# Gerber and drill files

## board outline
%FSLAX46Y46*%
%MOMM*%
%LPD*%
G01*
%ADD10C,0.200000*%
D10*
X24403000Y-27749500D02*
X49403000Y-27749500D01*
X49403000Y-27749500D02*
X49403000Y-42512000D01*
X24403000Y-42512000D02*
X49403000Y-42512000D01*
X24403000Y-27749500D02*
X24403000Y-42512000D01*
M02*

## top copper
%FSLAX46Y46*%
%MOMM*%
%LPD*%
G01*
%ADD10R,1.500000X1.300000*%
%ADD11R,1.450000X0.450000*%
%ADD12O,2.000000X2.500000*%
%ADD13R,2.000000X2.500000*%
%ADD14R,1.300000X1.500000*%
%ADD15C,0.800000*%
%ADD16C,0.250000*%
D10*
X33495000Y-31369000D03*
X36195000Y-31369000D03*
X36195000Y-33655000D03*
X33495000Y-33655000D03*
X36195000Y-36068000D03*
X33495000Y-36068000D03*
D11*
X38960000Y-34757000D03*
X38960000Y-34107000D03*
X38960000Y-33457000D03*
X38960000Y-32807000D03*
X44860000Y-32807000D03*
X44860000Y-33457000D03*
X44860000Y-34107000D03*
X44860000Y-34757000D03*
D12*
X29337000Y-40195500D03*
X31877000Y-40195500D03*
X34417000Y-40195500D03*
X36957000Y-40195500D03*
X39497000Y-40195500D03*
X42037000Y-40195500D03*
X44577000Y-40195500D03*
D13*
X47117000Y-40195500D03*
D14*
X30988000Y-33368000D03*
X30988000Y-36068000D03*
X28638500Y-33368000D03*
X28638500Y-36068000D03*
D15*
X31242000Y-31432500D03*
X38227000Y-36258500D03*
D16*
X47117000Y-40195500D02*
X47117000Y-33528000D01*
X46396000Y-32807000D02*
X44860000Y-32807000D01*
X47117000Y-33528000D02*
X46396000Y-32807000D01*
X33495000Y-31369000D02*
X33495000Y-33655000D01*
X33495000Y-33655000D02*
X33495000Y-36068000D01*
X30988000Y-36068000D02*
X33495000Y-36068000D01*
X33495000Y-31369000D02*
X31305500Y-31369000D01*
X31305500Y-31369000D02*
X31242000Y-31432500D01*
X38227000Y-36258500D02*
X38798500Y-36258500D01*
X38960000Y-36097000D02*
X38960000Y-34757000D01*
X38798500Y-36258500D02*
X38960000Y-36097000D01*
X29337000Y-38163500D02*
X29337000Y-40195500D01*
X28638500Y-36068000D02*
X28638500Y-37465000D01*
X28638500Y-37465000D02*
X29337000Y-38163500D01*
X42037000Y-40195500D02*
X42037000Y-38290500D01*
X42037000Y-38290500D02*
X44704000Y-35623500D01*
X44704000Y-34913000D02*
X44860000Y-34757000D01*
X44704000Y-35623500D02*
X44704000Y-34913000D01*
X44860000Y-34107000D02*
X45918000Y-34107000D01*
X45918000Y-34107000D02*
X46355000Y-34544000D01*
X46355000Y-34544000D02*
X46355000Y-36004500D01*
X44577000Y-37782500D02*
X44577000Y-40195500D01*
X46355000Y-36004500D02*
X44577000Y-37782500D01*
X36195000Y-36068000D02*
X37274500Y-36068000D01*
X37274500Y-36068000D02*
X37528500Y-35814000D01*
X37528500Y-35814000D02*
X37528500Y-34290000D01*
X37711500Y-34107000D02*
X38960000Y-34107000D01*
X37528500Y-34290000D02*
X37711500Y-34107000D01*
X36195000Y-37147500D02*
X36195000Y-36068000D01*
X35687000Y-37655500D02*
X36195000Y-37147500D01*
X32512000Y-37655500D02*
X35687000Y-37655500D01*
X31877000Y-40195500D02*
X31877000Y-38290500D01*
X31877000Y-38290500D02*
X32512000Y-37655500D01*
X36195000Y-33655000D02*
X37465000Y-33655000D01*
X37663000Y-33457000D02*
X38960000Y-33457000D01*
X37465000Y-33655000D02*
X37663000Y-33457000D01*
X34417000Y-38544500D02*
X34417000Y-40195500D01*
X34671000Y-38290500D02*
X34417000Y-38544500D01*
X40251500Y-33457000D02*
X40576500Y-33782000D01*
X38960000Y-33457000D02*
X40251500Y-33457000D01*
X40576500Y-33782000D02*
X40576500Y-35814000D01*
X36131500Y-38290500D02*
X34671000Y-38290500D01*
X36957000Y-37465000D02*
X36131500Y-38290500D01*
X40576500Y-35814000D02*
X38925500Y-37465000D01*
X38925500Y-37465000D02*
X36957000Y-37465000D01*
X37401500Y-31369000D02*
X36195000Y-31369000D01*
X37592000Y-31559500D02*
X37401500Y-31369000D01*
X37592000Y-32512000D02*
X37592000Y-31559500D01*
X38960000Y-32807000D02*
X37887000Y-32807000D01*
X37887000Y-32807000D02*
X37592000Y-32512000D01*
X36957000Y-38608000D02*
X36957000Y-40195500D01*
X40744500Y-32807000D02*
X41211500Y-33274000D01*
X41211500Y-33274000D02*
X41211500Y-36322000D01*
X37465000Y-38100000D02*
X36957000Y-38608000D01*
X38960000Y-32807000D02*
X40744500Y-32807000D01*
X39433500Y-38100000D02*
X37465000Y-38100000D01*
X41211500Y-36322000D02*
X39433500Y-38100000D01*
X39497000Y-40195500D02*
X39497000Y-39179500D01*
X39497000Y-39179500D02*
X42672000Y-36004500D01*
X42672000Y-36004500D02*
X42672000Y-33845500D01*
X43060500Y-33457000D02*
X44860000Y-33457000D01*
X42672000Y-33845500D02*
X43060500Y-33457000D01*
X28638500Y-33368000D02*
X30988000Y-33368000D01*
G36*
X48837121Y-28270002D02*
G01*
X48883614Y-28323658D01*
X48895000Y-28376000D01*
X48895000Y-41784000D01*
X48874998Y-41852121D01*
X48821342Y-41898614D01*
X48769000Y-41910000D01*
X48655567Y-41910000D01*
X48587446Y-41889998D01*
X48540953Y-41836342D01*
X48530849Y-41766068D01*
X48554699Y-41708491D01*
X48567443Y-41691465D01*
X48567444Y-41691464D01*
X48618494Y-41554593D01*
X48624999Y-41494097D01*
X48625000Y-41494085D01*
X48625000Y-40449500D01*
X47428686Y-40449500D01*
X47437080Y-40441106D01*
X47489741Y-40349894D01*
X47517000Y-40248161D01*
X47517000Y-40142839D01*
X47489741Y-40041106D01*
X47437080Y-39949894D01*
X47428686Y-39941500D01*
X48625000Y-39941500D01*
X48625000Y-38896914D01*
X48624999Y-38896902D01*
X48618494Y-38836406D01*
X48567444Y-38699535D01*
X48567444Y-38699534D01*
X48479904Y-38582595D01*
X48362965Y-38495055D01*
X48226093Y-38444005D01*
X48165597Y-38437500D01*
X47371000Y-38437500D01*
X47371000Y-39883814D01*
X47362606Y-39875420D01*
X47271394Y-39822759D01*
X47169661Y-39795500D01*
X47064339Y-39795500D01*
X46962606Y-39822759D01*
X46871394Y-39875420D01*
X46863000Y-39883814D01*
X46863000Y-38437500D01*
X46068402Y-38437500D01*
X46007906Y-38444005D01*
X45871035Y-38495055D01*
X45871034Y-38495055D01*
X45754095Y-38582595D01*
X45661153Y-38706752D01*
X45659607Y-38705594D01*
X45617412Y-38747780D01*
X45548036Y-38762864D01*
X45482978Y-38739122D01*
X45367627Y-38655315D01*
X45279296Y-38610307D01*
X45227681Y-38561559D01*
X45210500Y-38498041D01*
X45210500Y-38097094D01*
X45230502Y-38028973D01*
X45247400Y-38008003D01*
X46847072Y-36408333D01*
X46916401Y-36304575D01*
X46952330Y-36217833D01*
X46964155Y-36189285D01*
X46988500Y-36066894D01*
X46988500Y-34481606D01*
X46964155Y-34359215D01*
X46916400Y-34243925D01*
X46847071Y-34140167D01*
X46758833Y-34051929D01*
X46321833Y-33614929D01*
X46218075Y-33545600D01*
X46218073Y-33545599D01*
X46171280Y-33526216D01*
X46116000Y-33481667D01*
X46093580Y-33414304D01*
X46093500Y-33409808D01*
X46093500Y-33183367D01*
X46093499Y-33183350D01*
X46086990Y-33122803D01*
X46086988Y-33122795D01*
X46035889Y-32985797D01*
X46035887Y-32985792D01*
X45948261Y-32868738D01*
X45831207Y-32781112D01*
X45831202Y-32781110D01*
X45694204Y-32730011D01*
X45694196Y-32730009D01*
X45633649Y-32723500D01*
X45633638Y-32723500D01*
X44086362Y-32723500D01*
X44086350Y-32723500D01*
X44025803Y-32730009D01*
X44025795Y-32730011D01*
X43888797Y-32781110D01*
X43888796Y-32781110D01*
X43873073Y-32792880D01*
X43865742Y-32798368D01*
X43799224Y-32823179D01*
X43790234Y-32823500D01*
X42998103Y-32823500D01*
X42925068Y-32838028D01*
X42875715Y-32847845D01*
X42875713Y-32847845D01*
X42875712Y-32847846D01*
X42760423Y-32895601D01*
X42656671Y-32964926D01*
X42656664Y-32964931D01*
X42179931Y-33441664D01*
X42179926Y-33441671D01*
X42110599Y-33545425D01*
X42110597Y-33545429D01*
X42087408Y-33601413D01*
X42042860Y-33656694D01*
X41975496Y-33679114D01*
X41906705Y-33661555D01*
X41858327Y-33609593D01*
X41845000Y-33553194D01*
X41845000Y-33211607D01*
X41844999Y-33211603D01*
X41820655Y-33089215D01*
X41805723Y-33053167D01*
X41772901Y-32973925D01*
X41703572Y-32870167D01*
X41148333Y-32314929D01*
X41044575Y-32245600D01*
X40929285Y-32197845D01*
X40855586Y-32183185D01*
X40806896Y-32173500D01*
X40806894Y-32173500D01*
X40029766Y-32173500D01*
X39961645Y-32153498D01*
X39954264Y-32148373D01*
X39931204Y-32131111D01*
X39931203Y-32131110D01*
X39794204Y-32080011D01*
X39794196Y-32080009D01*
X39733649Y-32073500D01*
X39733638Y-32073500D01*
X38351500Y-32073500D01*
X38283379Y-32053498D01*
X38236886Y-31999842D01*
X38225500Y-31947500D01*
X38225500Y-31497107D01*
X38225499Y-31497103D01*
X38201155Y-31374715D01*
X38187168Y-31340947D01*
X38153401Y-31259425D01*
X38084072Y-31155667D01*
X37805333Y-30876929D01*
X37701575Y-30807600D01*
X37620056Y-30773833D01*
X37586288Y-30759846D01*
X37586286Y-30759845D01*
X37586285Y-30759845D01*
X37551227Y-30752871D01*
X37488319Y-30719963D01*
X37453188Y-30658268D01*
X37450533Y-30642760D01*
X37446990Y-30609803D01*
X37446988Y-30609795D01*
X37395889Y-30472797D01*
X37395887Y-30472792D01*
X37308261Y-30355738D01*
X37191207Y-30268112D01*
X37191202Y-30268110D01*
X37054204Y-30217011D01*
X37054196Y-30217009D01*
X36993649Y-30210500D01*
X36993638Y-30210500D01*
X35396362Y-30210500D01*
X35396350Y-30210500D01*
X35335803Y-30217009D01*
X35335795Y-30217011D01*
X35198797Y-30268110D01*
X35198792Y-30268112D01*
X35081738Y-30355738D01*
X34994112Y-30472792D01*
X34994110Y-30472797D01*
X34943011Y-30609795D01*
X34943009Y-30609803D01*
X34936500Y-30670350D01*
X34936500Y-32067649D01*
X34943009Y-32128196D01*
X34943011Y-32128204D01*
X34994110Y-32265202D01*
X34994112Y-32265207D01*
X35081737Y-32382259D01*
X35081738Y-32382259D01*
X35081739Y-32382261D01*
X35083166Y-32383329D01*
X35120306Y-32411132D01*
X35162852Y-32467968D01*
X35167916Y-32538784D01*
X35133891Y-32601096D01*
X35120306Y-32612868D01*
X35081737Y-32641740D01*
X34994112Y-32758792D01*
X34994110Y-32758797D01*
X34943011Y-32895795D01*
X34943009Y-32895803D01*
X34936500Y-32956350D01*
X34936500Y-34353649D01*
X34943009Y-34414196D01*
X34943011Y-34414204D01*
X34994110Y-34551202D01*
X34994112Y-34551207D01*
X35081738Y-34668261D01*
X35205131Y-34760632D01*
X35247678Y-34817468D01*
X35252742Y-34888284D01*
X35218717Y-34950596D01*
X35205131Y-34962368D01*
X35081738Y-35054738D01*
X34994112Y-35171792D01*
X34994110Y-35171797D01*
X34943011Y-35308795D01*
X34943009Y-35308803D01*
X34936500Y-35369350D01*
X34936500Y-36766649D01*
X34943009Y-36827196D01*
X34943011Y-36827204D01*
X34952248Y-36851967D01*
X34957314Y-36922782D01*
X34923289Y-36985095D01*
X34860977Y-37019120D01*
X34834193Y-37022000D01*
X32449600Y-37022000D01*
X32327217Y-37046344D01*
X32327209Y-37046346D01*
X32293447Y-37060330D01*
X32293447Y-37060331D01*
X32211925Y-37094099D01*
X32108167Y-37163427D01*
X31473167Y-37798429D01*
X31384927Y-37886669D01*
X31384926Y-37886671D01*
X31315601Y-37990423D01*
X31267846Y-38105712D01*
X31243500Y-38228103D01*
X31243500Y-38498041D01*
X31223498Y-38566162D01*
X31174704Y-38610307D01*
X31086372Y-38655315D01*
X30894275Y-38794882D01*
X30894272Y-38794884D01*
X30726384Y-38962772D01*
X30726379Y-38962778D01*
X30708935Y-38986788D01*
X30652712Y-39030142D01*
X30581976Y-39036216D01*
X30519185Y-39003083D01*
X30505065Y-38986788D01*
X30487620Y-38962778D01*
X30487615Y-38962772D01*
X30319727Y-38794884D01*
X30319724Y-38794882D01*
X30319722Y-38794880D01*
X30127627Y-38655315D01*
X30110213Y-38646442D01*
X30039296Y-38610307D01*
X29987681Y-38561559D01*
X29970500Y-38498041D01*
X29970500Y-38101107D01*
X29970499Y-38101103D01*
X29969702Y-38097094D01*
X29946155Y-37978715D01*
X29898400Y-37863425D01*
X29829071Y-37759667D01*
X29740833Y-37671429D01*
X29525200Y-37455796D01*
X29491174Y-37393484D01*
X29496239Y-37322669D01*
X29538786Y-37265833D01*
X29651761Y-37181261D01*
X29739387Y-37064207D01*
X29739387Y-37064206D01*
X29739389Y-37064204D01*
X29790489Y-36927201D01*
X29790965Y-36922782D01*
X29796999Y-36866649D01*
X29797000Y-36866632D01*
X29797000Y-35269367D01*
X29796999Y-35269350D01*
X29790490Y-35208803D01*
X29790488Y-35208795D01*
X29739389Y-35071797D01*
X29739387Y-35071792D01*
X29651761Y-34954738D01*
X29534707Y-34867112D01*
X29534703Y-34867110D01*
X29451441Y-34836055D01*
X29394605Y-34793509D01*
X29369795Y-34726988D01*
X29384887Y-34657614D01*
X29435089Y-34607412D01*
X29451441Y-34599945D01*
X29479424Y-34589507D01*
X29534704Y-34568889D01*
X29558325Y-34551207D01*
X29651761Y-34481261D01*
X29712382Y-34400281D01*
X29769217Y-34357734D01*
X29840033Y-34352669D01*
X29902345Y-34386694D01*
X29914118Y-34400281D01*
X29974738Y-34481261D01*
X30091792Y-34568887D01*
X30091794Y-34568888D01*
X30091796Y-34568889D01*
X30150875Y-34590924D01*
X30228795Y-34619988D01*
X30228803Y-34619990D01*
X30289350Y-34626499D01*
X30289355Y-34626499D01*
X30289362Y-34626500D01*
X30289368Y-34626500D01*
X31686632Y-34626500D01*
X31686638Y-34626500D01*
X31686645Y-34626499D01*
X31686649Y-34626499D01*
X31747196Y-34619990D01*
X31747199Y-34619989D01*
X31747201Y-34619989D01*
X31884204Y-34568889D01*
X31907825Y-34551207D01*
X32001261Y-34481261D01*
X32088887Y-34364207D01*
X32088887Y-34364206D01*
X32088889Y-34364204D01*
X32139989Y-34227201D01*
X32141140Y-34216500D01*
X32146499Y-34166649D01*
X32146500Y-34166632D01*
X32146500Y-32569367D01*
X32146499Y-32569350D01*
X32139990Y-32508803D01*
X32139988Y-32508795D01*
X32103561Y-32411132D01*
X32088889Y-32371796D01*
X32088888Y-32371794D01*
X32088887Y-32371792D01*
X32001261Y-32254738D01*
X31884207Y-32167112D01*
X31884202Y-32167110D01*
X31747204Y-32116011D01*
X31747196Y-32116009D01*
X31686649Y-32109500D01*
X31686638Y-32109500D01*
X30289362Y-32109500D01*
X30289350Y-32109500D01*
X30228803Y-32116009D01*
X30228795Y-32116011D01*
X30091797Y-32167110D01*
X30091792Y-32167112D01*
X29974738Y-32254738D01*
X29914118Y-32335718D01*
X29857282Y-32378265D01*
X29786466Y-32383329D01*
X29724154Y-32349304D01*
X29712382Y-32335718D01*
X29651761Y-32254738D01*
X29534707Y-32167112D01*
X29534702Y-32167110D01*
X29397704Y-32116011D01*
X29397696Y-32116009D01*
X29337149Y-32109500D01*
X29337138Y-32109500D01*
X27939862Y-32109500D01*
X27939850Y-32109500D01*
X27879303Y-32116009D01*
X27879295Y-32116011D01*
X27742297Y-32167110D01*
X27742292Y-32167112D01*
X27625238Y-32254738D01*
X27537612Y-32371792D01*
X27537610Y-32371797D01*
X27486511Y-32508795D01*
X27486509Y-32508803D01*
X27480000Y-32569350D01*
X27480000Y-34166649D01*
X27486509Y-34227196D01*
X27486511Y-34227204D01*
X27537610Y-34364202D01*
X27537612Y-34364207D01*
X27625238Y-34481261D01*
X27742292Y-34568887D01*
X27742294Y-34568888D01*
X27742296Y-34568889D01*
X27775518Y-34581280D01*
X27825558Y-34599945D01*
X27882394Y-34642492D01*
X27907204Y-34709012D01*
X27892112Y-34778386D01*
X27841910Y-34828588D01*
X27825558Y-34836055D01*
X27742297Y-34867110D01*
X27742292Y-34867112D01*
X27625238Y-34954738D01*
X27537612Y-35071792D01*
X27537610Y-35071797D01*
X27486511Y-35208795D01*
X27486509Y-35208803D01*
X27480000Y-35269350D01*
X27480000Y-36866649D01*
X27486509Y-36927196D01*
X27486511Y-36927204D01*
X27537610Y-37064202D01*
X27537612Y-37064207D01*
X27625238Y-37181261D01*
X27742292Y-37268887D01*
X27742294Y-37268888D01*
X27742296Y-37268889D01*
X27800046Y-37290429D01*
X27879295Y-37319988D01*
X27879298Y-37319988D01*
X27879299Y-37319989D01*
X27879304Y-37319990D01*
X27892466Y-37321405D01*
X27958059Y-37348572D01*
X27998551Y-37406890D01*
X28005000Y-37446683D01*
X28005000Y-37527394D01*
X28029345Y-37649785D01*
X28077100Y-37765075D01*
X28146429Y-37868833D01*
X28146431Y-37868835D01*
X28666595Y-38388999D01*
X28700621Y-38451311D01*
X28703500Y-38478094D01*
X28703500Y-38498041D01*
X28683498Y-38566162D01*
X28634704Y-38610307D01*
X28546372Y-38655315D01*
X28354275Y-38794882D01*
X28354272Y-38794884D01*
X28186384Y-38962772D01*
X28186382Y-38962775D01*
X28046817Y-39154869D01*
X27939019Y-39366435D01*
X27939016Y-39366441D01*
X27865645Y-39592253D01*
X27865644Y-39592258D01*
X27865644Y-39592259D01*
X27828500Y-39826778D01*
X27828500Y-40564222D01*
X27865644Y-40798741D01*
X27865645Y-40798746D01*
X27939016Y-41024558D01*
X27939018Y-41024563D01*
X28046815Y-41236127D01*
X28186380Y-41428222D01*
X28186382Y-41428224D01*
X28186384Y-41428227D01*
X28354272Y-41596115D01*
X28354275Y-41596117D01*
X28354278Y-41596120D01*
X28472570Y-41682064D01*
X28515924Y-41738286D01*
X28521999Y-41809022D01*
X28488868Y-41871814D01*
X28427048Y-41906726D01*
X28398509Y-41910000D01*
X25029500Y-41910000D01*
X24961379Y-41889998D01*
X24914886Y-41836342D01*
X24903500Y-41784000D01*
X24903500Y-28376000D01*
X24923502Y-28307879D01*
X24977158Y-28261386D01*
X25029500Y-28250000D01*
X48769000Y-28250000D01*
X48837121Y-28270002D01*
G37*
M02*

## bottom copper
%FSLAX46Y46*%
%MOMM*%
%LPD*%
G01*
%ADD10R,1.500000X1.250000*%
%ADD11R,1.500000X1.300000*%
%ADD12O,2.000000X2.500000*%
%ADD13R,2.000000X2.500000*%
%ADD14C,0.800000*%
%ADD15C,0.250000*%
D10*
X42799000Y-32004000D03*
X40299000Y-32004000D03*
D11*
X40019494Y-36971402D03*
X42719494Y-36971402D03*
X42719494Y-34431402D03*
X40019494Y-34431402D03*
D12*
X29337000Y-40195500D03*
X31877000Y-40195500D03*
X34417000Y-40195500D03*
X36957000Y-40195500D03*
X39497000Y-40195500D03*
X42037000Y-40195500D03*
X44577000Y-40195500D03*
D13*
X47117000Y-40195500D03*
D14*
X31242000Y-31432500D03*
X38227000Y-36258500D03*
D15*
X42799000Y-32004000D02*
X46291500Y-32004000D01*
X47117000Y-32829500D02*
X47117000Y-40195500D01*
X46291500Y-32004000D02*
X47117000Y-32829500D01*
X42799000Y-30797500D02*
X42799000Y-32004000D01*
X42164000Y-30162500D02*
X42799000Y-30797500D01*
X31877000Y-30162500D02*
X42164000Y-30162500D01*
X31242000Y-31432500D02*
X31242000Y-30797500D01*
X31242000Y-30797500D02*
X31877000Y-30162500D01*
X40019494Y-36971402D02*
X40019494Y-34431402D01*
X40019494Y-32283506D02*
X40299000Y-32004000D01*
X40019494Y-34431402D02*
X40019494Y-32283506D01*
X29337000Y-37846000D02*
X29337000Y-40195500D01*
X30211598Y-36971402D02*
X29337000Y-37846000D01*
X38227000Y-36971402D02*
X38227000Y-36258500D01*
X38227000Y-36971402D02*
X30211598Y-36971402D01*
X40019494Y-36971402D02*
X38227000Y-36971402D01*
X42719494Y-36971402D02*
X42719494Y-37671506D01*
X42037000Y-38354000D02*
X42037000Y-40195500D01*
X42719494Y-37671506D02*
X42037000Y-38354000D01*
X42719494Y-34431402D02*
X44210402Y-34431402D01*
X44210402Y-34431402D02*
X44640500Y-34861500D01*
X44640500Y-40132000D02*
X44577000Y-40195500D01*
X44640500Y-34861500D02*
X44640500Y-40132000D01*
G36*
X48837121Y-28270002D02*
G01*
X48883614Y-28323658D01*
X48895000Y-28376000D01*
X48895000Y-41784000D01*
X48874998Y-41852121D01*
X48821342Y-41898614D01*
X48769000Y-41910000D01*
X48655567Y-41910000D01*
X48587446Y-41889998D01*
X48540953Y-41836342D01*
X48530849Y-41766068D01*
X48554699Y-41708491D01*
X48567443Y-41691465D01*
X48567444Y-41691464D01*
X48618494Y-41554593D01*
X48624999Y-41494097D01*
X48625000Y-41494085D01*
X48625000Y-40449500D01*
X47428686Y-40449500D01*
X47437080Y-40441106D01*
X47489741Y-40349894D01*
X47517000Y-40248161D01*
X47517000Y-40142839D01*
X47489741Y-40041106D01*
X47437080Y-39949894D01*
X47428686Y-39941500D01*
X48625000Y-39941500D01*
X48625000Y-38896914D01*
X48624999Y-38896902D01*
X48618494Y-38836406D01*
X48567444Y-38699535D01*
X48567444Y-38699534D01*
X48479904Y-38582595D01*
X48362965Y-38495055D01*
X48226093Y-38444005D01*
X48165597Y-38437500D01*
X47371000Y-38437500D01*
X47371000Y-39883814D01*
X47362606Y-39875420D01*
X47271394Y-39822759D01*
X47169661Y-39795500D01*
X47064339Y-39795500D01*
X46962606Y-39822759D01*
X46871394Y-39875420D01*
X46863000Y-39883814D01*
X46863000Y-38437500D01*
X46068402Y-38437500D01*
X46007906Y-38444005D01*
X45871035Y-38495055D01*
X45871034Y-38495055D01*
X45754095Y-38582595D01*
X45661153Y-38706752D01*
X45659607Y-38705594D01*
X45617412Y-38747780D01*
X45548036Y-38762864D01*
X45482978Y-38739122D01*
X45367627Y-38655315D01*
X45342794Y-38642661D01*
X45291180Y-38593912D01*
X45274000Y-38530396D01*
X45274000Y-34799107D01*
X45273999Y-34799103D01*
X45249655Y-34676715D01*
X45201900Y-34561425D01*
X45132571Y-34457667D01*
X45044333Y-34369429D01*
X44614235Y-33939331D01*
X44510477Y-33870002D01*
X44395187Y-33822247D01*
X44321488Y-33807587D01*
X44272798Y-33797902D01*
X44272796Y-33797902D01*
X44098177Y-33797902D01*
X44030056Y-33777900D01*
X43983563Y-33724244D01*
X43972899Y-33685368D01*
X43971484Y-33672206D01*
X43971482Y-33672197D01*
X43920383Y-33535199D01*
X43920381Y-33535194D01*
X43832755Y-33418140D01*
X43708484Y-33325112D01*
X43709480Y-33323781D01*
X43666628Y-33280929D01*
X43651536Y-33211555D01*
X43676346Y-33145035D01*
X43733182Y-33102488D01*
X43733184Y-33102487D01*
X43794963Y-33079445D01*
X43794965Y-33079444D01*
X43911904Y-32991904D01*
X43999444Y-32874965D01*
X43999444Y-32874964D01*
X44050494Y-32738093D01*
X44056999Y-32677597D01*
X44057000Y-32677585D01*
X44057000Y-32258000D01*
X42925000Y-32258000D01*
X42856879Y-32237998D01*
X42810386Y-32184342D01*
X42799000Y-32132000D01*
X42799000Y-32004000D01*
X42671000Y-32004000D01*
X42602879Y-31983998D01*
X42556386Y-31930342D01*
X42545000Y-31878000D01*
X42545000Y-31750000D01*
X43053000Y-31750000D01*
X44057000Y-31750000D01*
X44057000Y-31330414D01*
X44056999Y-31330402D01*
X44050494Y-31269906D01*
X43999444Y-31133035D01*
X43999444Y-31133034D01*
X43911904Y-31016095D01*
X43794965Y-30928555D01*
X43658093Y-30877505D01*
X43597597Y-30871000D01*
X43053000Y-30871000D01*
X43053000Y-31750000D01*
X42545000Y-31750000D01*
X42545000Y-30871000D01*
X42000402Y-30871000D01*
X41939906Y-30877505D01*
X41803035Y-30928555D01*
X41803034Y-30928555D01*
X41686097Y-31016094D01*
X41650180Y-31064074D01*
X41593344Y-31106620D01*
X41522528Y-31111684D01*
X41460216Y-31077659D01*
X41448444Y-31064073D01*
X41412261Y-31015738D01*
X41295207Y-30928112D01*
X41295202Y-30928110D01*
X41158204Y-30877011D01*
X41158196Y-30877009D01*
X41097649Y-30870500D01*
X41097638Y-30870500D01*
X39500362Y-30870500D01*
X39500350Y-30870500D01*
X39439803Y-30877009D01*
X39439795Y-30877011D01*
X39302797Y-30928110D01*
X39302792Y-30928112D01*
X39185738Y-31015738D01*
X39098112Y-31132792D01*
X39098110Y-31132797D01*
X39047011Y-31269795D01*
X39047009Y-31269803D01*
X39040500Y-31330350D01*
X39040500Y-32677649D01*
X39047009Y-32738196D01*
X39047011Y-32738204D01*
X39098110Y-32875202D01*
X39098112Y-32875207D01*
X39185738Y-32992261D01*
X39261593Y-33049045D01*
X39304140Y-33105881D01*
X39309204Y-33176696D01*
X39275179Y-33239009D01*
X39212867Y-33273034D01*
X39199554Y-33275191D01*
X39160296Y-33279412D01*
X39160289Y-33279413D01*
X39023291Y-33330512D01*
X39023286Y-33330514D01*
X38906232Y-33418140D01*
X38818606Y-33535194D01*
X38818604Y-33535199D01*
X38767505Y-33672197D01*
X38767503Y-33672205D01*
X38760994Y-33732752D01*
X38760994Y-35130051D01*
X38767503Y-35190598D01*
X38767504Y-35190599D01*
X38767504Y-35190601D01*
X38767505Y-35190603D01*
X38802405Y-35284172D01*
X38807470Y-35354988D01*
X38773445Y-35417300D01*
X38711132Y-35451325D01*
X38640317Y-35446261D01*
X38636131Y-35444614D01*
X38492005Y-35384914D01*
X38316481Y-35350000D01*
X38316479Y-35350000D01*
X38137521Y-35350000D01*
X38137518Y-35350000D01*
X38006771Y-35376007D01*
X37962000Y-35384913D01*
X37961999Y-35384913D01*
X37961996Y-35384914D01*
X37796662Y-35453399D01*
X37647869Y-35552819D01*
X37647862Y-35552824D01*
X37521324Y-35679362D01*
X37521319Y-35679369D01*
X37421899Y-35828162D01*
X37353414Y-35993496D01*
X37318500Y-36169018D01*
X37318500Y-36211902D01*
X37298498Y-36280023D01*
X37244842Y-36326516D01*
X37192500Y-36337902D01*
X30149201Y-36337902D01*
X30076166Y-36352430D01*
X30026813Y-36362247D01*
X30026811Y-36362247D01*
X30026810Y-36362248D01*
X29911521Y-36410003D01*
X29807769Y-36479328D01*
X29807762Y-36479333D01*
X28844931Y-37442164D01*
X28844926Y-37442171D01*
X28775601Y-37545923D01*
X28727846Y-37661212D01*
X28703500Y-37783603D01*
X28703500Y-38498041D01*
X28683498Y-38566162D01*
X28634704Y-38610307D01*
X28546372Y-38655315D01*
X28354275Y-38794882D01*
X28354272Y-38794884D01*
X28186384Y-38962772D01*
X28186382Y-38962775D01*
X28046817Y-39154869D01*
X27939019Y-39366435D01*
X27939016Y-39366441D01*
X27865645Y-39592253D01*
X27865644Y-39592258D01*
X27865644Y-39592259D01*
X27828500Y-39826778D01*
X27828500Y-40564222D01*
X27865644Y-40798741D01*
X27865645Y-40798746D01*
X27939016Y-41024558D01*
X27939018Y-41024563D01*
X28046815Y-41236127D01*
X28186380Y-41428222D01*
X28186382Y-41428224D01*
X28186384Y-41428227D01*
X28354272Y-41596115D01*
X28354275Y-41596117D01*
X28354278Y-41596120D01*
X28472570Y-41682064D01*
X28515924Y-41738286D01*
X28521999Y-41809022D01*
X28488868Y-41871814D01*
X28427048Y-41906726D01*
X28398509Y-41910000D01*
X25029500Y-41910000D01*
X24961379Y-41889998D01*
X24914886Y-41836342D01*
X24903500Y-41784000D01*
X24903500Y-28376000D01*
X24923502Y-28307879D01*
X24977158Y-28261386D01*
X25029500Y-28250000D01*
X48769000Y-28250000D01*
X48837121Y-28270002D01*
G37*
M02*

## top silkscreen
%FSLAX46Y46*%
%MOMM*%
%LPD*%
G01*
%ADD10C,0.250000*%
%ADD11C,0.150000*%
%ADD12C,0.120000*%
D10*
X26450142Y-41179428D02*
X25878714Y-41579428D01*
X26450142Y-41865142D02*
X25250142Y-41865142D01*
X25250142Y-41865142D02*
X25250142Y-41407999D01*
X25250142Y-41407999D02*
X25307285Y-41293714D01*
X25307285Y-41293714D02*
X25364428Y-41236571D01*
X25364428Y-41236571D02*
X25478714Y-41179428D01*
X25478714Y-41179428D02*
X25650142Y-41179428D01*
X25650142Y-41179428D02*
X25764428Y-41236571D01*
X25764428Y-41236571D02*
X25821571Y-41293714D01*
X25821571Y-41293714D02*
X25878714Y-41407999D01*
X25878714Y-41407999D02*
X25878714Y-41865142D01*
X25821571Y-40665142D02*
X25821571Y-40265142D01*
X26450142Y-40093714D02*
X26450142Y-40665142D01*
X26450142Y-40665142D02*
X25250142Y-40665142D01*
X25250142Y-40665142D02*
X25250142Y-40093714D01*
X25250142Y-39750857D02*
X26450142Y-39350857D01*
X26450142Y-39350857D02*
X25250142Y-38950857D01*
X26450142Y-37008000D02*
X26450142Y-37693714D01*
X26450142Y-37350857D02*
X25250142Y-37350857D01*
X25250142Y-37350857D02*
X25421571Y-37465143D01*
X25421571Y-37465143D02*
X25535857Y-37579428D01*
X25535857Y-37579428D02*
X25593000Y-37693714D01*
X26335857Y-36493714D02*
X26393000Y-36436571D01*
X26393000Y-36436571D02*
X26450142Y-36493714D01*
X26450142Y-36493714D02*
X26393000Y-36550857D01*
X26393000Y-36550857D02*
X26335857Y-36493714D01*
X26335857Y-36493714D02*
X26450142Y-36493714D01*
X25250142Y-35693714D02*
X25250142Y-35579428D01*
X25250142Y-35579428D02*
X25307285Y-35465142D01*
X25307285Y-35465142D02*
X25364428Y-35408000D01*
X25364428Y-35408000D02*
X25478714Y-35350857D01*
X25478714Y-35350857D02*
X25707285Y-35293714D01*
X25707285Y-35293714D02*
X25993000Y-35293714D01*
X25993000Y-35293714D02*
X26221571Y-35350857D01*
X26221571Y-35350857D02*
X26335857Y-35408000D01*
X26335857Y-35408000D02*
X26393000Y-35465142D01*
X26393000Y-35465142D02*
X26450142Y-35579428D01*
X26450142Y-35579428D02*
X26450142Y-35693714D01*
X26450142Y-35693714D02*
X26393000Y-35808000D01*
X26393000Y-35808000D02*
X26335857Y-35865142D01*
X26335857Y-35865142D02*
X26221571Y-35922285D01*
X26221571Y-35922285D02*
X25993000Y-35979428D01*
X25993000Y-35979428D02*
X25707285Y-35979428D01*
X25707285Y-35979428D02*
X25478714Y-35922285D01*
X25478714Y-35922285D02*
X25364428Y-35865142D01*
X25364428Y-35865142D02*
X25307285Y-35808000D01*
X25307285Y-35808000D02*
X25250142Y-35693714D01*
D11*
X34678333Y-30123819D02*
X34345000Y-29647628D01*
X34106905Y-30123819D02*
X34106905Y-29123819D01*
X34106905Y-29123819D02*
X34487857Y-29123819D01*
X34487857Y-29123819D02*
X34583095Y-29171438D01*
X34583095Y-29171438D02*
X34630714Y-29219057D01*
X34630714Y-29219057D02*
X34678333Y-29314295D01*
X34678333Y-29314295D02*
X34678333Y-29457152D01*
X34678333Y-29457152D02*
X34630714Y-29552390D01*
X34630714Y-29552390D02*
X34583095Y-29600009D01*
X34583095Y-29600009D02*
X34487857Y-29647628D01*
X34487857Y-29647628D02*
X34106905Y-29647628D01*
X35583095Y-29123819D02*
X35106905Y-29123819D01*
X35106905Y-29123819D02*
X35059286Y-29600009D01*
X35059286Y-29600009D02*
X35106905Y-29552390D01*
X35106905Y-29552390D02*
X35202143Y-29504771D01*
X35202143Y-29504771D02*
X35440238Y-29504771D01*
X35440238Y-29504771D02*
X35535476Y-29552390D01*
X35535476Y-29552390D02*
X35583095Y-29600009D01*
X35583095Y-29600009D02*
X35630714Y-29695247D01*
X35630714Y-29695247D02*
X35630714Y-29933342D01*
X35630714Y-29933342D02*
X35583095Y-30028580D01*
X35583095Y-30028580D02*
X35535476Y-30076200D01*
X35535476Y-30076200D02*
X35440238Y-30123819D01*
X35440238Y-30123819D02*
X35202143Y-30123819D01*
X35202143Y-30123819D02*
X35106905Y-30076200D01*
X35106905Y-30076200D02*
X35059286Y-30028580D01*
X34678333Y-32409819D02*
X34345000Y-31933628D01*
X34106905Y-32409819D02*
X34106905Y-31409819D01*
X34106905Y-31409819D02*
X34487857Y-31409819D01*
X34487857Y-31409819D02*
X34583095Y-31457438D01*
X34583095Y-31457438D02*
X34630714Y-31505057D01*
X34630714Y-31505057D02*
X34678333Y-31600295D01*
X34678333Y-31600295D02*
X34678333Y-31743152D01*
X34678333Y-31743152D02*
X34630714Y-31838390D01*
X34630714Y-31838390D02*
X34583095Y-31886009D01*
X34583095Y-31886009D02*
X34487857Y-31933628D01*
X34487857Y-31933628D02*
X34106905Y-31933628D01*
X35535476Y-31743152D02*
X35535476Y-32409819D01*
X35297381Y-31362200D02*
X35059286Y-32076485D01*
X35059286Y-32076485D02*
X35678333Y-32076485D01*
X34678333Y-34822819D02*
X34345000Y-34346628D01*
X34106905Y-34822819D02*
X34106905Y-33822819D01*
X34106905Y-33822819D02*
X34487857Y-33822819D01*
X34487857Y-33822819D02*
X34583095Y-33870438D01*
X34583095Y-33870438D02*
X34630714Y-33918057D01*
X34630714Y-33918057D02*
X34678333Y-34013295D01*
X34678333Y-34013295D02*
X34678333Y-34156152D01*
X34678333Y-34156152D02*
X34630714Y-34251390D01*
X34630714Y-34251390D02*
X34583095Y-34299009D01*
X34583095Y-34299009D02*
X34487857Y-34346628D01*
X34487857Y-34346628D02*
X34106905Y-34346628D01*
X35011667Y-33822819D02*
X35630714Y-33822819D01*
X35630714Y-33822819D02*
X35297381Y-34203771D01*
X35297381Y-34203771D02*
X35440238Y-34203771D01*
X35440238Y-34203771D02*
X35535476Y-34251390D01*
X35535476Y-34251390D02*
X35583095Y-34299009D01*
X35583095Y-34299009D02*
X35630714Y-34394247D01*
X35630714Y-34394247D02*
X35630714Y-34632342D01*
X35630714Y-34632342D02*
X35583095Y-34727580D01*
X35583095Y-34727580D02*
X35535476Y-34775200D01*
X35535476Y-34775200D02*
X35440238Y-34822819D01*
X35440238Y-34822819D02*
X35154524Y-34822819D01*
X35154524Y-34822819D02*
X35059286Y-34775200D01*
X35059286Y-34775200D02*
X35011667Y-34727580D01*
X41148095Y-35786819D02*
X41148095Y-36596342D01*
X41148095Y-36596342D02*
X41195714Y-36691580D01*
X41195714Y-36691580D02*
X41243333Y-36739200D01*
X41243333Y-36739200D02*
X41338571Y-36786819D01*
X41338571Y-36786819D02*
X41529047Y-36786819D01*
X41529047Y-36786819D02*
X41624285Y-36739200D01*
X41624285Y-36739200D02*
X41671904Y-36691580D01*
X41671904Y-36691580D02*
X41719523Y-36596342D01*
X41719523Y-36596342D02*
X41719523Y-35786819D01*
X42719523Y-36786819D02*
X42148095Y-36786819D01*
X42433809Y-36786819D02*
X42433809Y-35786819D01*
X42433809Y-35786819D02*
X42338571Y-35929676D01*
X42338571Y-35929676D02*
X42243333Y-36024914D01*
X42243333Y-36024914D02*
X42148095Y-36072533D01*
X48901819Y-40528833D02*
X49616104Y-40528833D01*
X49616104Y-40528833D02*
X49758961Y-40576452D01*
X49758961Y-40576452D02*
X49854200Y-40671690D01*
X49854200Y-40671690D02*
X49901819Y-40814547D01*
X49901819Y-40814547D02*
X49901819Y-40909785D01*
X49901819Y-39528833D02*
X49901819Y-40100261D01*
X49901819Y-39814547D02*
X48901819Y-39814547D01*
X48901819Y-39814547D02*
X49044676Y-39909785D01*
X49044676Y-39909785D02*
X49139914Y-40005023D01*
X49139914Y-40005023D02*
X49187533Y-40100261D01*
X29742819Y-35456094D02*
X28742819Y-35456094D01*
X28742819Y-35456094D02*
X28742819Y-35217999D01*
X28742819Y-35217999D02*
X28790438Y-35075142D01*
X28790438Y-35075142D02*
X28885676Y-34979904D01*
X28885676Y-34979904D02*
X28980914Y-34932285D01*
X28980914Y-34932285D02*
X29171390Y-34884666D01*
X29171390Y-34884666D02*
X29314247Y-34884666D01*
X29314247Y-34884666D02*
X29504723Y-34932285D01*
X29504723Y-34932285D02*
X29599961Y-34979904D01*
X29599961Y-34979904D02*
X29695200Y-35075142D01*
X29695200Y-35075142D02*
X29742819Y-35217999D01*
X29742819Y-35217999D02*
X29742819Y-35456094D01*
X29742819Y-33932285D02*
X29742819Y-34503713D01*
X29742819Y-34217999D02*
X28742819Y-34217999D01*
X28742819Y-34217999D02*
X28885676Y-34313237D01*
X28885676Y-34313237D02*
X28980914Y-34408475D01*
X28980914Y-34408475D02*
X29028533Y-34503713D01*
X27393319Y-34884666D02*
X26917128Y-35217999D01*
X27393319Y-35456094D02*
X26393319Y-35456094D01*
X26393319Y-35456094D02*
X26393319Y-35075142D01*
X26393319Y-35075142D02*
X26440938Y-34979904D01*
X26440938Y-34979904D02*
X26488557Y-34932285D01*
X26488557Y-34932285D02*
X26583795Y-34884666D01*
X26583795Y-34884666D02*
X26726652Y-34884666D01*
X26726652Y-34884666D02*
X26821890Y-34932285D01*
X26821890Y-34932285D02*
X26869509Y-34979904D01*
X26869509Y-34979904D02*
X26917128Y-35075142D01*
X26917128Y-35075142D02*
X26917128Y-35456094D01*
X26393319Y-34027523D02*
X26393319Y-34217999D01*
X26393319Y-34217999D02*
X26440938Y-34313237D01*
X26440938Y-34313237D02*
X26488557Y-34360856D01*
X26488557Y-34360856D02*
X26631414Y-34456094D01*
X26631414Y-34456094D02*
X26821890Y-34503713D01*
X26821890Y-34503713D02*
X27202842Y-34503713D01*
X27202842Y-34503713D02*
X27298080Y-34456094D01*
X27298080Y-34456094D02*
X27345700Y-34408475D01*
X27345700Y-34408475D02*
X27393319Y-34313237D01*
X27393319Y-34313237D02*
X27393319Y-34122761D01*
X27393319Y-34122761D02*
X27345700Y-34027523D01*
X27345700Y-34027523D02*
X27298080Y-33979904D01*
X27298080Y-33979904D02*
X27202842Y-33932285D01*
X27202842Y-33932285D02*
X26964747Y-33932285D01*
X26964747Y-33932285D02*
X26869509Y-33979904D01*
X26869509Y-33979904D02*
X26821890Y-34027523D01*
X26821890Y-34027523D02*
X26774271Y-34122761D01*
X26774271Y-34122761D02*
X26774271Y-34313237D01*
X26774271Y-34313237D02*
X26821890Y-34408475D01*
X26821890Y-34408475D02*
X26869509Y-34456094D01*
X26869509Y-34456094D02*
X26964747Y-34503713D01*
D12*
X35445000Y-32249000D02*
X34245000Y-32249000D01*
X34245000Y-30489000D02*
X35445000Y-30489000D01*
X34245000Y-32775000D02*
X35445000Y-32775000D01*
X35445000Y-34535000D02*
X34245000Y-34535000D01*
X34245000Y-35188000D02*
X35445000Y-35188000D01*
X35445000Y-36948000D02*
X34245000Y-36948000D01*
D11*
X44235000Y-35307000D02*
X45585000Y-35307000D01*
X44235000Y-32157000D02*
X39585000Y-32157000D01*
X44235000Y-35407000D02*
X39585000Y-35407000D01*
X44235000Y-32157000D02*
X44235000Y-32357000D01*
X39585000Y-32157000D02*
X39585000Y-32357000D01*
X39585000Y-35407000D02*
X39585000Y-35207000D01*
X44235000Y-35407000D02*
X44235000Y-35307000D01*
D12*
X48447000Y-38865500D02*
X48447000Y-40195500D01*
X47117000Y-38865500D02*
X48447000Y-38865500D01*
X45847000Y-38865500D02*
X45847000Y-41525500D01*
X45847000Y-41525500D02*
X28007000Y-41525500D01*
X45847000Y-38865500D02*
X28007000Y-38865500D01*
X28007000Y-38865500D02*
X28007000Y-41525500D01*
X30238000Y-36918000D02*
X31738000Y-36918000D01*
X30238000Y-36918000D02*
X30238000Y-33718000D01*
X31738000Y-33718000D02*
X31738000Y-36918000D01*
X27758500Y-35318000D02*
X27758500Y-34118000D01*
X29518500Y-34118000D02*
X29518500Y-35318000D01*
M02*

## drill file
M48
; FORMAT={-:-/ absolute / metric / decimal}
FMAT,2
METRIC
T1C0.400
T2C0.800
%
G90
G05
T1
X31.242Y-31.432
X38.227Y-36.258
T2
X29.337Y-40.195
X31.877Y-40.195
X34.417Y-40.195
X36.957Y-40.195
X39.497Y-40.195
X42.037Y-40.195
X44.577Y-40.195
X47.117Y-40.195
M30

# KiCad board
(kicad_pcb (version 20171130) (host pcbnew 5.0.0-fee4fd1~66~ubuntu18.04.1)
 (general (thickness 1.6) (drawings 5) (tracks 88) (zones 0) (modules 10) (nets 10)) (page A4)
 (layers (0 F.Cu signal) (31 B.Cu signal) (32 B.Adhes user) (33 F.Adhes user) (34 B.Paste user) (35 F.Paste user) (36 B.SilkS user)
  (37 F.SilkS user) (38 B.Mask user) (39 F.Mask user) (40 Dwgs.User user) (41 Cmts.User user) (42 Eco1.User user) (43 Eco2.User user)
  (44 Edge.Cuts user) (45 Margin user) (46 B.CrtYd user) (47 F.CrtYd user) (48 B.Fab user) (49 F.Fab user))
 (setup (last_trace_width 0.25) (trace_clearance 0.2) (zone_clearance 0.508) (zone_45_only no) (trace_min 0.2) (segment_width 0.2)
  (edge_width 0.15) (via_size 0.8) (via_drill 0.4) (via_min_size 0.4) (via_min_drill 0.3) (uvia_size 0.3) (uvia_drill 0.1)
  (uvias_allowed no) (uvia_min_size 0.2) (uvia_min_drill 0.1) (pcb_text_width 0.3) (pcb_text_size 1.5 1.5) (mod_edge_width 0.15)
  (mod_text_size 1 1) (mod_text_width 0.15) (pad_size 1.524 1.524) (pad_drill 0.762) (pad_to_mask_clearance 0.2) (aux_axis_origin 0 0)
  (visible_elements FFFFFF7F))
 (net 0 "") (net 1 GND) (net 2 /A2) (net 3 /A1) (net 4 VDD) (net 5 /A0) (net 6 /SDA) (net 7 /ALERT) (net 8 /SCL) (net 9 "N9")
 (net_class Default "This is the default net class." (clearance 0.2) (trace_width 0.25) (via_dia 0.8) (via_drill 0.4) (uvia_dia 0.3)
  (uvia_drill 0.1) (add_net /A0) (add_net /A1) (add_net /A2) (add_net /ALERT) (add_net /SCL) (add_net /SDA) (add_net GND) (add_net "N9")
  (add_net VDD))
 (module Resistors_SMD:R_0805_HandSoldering (layer F.Cu) (at 34.845 31.369)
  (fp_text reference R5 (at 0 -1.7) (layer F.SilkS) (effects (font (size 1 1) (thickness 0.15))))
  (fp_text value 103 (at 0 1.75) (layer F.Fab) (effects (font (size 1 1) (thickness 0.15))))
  (fp_line (start 0.6 0.88) (end -0.6 0.88) (layer F.SilkS) (width 0.12))
  (fp_line (start -0.6 -0.88) (end 0.6 -0.88) (layer F.SilkS) (width 0.12))
  (pad 1 smd rect (at -1.35 0) (size 1.5 1.3) (layers F.Cu F.Paste F.Mask) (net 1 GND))
  (pad 2 smd rect (at 1.35 0) (size 1.5 1.3) (layers F.Cu F.Paste F.Mask) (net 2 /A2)))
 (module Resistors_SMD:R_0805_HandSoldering (layer F.Cu) (at 34.845 33.655)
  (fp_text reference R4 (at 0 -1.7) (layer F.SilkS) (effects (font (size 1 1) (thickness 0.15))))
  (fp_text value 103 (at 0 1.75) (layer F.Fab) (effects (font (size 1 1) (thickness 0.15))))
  (fp_line (start -0.6 -0.88) (end 0.6 -0.88) (layer F.SilkS) (width 0.12))
  (fp_line (start 0.6 0.88) (end -0.6 0.88) (layer F.SilkS) (width 0.12))
  (pad 2 smd rect (at 1.35 0) (size 1.5 1.3) (layers F.Cu F.Paste F.Mask) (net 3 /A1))
  (pad 1 smd rect (at -1.35 0) (size 1.5 1.3) (layers F.Cu F.Paste F.Mask) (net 1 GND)))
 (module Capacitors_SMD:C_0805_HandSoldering (layer B.Cu) (at 41.549 32.004)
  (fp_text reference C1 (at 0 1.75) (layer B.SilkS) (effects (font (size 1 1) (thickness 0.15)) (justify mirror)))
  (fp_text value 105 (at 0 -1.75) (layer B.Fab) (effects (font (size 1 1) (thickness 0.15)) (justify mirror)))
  (pad 2 smd rect (at 1.25 0) (size 1.5 1.25) (layers B.Cu B.Paste B.Mask) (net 1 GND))
  (pad 1 smd rect (at -1.25 0) (size 1.5 1.25) (layers B.Cu B.Paste B.Mask) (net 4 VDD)))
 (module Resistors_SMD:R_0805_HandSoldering (layer F.Cu) (at 34.845 36.068)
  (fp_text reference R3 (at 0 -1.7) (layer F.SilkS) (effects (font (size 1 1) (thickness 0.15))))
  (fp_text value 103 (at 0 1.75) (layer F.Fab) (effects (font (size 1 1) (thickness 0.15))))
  (fp_line (start -0.6 -0.88) (end 0.6 -0.88) (layer F.SilkS) (width 0.12))
  (fp_line (start 0.6 0.88) (end -0.6 0.88) (layer F.SilkS) (width 0.12))
  (pad 2 smd rect (at 1.35 0) (size 1.5 1.3) (layers F.Cu F.Paste F.Mask) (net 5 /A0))
  (pad 1 smd rect (at -1.35 0) (size 1.5 1.3) (layers F.Cu F.Paste F.Mask) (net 1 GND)))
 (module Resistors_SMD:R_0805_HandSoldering (layer B.Cu) (at 41.369494 36.971402 180)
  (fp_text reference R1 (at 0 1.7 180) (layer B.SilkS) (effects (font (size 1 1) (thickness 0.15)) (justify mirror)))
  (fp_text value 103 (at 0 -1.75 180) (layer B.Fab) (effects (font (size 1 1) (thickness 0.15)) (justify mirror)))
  (pad 2 smd rect (at 1.35 0 180) (size 1.5 1.3) (layers B.Cu B.Paste B.Mask) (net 4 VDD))
  (pad 1 smd rect (at -1.35 0 180) (size 1.5 1.3) (layers B.Cu B.Paste B.Mask) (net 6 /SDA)))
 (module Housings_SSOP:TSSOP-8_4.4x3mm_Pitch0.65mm (layer F.Cu) (at 41.91 33.782 180)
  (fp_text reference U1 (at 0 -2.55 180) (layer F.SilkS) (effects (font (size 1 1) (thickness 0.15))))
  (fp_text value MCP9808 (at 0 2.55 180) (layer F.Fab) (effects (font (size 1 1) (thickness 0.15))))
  (fp_line (start -2.325 -1.525) (end -3.675 -1.525) (layer F.SilkS) (width 0.15))
  (fp_line (start -2.325 1.625) (end 2.325 1.625) (layer F.SilkS) (width 0.15))
  (fp_line (start -2.325 -1.625) (end 2.325 -1.625) (layer F.SilkS) (width 0.15))
  (fp_line (start -2.325 1.625) (end -2.325 1.425) (layer F.SilkS) (width 0.15))
  (fp_line (start 2.325 1.625) (end 2.325 1.425) (layer F.SilkS) (width 0.15))
  (fp_line (start 2.325 -1.625) (end 2.325 -1.425) (layer F.SilkS) (width 0.15))
  (fp_line (start -2.325 -1.625) (end -2.325 -1.525) (layer F.SilkS) (width 0.15))
  (pad 8 smd rect (at 2.95 -0.975 180) (size 1.45 0.45) (layers F.Cu F.Paste F.Mask) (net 4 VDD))
  (pad 7 smd rect (at 2.95 -0.325 180) (size 1.45 0.45) (layers F.Cu F.Paste F.Mask) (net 5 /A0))
  (pad 6 smd rect (at 2.95 0.325 180) (size 1.45 0.45) (layers F.Cu F.Paste F.Mask) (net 3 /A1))
  (pad 5 smd rect (at 2.95 0.975 180) (size 1.45 0.45) (layers F.Cu F.Paste F.Mask) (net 2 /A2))
  (pad 4 smd rect (at -2.95 0.975 180) (size 1.45 0.45) (layers F.Cu F.Paste F.Mask) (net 1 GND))
  (pad 3 smd rect (at -2.95 0.325 180) (size 1.45 0.45) (layers F.Cu F.Paste F.Mask) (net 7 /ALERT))
  (pad 2 smd rect (at -2.95 -0.325 180) (size 1.45 0.45) (layers F.Cu F.Paste F.Mask) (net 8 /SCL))
  (pad 1 smd rect (at -2.95 -0.975 180) (size 1.45 0.45) (layers F.Cu F.Paste F.Mask) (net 6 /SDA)))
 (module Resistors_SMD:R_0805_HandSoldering (layer B.Cu) (at 41.369494 34.431402 180)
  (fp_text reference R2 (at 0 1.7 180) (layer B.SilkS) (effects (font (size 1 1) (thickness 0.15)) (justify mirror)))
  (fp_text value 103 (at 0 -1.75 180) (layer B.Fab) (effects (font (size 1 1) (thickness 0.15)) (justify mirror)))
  (pad 1 smd rect (at -1.35 0 180) (size 1.5 1.3) (layers B.Cu B.Paste B.Mask) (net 8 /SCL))
  (pad 2 smd rect (at 1.35 0 180) (size 1.5 1.3) (layers B.Cu B.Paste B.Mask) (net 4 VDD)))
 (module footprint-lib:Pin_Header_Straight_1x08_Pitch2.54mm (layer F.Cu) (at 47.117 40.1955 270)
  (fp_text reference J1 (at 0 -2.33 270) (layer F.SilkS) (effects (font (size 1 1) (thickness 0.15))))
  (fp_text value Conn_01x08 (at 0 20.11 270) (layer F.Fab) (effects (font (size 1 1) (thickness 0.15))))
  (fp_line (start -1.33 -1.33) (end 0 -1.33) (layer F.SilkS) (width 0.12))
  (fp_line (start -1.33 0) (end -1.33 -1.33) (layer F.SilkS) (width 0.12))
  (fp_line (start -1.33 1.27) (end 1.33 1.27) (layer F.SilkS) (width 0.12))
  (fp_line (start 1.33 1.27) (end 1.33 19.11) (layer F.SilkS) (width 0.12))
  (fp_line (start -1.33 1.27) (end -1.33 19.11) (layer F.SilkS) (width 0.12))
  (fp_line (start -1.33 19.11) (end 1.33 19.11) (layer F.SilkS) (width 0.12))
  (pad 8 thru_hole oval (at 0 17.78 270) (size 2.5 2) (drill 0.8) (layers *.Cu *.Mask) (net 4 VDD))
  (pad 7 thru_hole oval (at 0 15.24 270) (size 2.5 2) (drill 0.8) (layers *.Cu *.Mask) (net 5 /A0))
  (pad 6 thru_hole oval (at 0 12.7 270) (size 2.5 2) (drill 0.8) (layers *.Cu *.Mask) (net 3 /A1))
  (pad 5 thru_hole oval (at 0 10.16 270) (size 2.5 2) (drill 0.8) (layers *.Cu *.Mask) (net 2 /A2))
  (pad 4 thru_hole oval (at 0 7.62 270) (size 2.5 2) (drill 0.8) (layers *.Cu *.Mask) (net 7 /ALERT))
  (pad 3 thru_hole oval (at 0 5.08 270) (size 2.5 2) (drill 0.8) (layers *.Cu *.Mask) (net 6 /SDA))
  (pad 2 thru_hole oval (at 0 2.54 270) (size 2.5 2) (drill 0.8) (layers *.Cu *.Mask) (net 8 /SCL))
  (pad 1 thru_hole rect (at 0 0 270) (size 2.5 2) (drill 0.8) (layers *.Cu *.Mask) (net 1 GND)))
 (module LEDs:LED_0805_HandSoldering (layer F.Cu) (at 30.988 34.718 90)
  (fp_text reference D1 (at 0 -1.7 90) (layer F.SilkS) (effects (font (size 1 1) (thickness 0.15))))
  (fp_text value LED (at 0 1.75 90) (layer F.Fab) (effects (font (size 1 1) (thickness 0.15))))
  (fp_line (start -2.2 -0.75) (end -2.2 0.75) (layer F.SilkS) (width 0.12))
  (fp_line (start -2.2 -0.75) (end 1 -0.75) (layer F.SilkS) (width 0.12))
  (fp_line (start 1 0.75) (end -2.2 0.75) (layer F.SilkS) (width 0.12))
  (pad 2 smd rect (at 1.35 0 90) (size 1.5 1.3) (layers F.Cu F.Paste F.Mask) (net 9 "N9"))
  (pad 1 smd rect (at -1.35 0 90) (size 1.5 1.3) (layers F.Cu F.Paste F.Mask) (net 1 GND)))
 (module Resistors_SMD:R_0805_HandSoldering (layer F.Cu) (at 28.6385 34.718 90)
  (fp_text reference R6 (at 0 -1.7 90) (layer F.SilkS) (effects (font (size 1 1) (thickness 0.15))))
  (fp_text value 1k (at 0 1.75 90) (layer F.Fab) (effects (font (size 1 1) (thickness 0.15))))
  (fp_line (start -0.6 -0.88) (end 0.6 -0.88) (layer F.SilkS) (width 0.12))
  (fp_line (start 0.6 0.88) (end -0.6 0.88) (layer F.SilkS) (width 0.12))
  (pad 2 smd rect (at 1.35 0 90) (size 1.5 1.3) (layers F.Cu F.Paste F.Mask) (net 9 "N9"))
  (pad 1 smd rect (at -1.35 0 90) (size 1.5 1.3) (layers F.Cu F.Paste F.Mask) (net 4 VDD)))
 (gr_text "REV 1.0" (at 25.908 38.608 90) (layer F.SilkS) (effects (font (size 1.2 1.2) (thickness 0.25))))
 (gr_line (start 24.403 27.7495) (end 49.403 27.7495) (layer Edge.Cuts) (width 0.2))
 (gr_line (start 49.403 27.7495) (end 49.403 42.512) (layer Edge.Cuts) (width 0.2))
 (gr_line (start 24.403 42.512) (end 49.403 42.512) (layer Edge.Cuts) (width 0.2))
 (gr_line (start 24.403 27.7495) (end 24.403 42.512) (layer Edge.Cuts) (width 0.2))
 (segment (start 47.117 40.1955) (end 47.117 33.528) (width 0.25) (layer F.Cu) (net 1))
 (segment (start 46.396 32.807) (end 44.86 32.807) (width 0.25) (layer F.Cu) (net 1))
 (segment (start 47.117 33.528) (end 46.396 32.807) (width 0.25) (layer F.Cu) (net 1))
 (segment (start 33.495 31.369) (end 33.495 33.655) (width 0.25) (layer F.Cu) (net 1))
 (segment (start 33.495 33.655) (end 33.495 36.068) (width 0.25) (layer F.Cu) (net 1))
 (segment (start 30.988 36.068) (end 33.495 36.068) (width 0.25) (layer F.Cu) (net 1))
 (segment (start 42.799 32.004) (end 46.2915 32.004) (width 0.25) (layer B.Cu) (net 1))
 (segment (start 47.117 32.8295) (end 47.117 40.1955) (width 0.25) (layer B.Cu) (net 1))
 (segment (start 46.2915 32.004) (end 47.117 32.8295) (width 0.25) (layer B.Cu) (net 1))
 (via (at 31.242 31.4325) (size 0.8) (drill 0.4) (layers F.Cu B.Cu) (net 1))
 (segment (start 33.495 31.369) (end 31.3055 31.369) (width 0.25) (layer F.Cu) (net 1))
 (segment (start 31.3055 31.369) (end 31.242 31.4325) (width 0.25) (layer F.Cu) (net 1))
 (segment (start 42.799 30.7975) (end 42.799 32.004) (width 0.25) (layer B.Cu) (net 1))
 (segment (start 42.164 30.1625) (end 42.799 30.7975) (width 0.25) (layer B.Cu) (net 1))
 (segment (start 31.877 30.1625) (end 42.164 30.1625) (width 0.25) (layer B.Cu) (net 1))
 (segment (start 31.242 31.4325) (end 31.242 30.7975) (width 0.25) (layer B.Cu) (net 1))
 (segment (start 31.242 30.7975) (end 31.877 30.1625) (width 0.25) (layer B.Cu) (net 1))
 (segment (start 40.019494 36.971402) (end 40.019494 34.431402) (width 0.25) (layer B.Cu) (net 4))
 (segment (start 40.019494 32.283506) (end 40.299 32.004) (width 0.25) (layer B.Cu) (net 4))
 (segment (start 40.019494 34.431402) (end 40.019494 32.283506) (width 0.25) (layer B.Cu) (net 4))
 (segment (start 29.337 37.846) (end 29.337 40.1955) (width 0.25) (layer B.Cu) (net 4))
 (segment (start 30.211598 36.971402) (end 29.337 37.846) (width 0.25) (layer B.Cu) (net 4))
 (via (at 38.227 36.2585) (size 0.8) (drill 0.4) (layers F.Cu B.Cu) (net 4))
 (segment (start 38.227 36.971402) (end 38.227 36.2585) (width 0.25) (layer B.Cu) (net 4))
 (segment (start 38.227 36.971402) (end 30.211598 36.971402) (width 0.25) (layer B.Cu) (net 4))
 (segment (start 40.019494 36.971402) (end 38.227 36.971402) (width 0.25) (layer B.Cu) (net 4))
 (segment (start 38.227 36.2585) (end 38.7985 36.2585) (width 0.25) (layer F.Cu) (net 4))
 (segment (start 38.96 36.097) (end 38.96 34.757) (width 0.25) (layer F.Cu) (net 4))
 (segment (start 38.7985 36.2585) (end 38.96 36.097) (width 0.25) (layer F.Cu) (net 4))
 (segment (start 29.337 38.1635) (end 29.337 40.1955) (width 0.25) (layer F.Cu) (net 4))
 (segment (start 28.6385 36.068) (end 28.6385 37.465) (width 0.25) (layer F.Cu) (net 4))
 (segment (start 28.6385 37.465) (end 29.337 38.1635) (width 0.25) (layer F.Cu) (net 4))
 (segment (start 42.719494 36.971402) (end 42.719494 37.671506) (width 0.25) (layer B.Cu) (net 6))
 (segment (start 42.037 38.354) (end 42.037 40.1955) (width 0.25) (layer B.Cu) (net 6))
 (segment (start 42.719494 37.671506) (end 42.037 38.354) (width 0.25) (layer B.Cu) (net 6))
 (segment (start 42.037 40.1955) (end 42.037 38.2905) (width 0.25) (layer F.Cu) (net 6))
 (segment (start 42.037 38.2905) (end 44.704 35.6235) (width 0.25) (layer F.Cu) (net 6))
 (segment (start 44.704 34.913) (end 44.86 34.757) (width 0.25) (layer F.Cu) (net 6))
 (segment (start 44.704 35.6235) (end 44.704 34.913) (width 0.25) (layer F.Cu) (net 6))
 (segment (start 42.719494 34.431402) (end 44.210402 34.431402) (width 0.25) (layer B.Cu) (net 8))
 (segment (start 44.210402 34.431402) (end 44.6405 34.8615) (width 0.25) (layer B.Cu) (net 8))
 (segment (start 44.6405 40.132) (end 44.577 40.1955) (width 0.25) (layer B.Cu) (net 8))
 (segment (start 44.6405 34.8615) (end 44.6405 40.132) (width 0.25) (layer B.Cu) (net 8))
 (segment (start 44.86 34.107) (end 45.918 34.107) (width 0.25) (layer F.Cu) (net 8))
 (segment (start 45.918 34.107) (end 46.355 34.544) (width 0.25) (layer F.Cu) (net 8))
 (segment (start 46.355 34.544) (end 46.355 36.0045) (width 0.25) (layer F.Cu) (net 8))
 (segment (start 44.577 37.7825) (end 44.577 40.1955) (width 0.25) (layer F.Cu) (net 8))
 (segment (start 46.355 36.0045) (end 44.577 37.7825) (width 0.25) (layer F.Cu) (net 8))
 (segment (start 36.195 36.068) (end 37.2745 36.068) (width 0.25) (layer F.Cu) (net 5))
 (segment (start 37.2745 36.068) (end 37.5285 35.814) (width 0.25) (layer F.Cu) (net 5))
 (segment (start 37.5285 35.814) (end 37.5285 34.29) (width 0.25) (layer F.Cu) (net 5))
 (segment (start 37.7115 34.107) (end 38.96 34.107) (width 0.25) (layer F.Cu) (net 5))
 (segment (start 37.5285 34.29) (end 37.7115 34.107) (width 0.25) (layer F.Cu) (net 5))
 (segment (start 36.195 37.1475) (end 36.195 36.068) (width 0.25) (layer F.Cu) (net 5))
 (segment (start 35.687 37.6555) (end 36.195 37.1475) (width 0.25) (layer F.Cu) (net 5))
 (segment (start 32.512 37.6555) (end 35.687 37.6555) (width 0.25) (layer F.Cu) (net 5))
 (segment (start 31.877 40.1955) (end 31.877 38.2905) (width 0.25) (layer F.Cu) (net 5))
 (segment (start 31.877 38.2905) (end 32.512 37.6555) (width 0.25) (layer F.Cu) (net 5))
 (segment (start 36.195 33.655) (end 37.465 33.655) (width 0.25) (layer F.Cu) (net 3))
 (segment (start 37.663 33.457) (end 38.96 33.457) (width 0.25) (layer F.Cu) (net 3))
 (segment (start 37.465 33.655) (end 37.663 33.457) (width 0.25) (layer F.Cu) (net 3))
 (segment (start 34.417 38.5445) (end 34.417 40.1955) (width 0.25) (layer F.Cu) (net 3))
 (segment (start 34.671 38.2905) (end 34.417 38.5445) (width 0.25) (layer F.Cu) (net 3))
 (segment (start 40.2515 33.457) (end 40.5765 33.782) (width 0.25) (layer F.Cu) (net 3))
 (segment (start 38.96 33.457) (end 40.2515 33.457) (width 0.25) (layer F.Cu) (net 3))
 (segment (start 40.5765 33.782) (end 40.5765 35.814) (width 0.25) (layer F.Cu) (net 3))
 (segment (start 36.1315 38.2905) (end 34.671 38.2905) (width 0.25) (layer F.Cu) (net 3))
 (segment (start 36.957 37.465) (end 36.1315 38.2905) (width 0.25) (layer F.Cu) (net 3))
 (segment (start 40.5765 35.814) (end 38.9255 37.465) (width 0.25) (layer F.Cu) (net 3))
 (segment (start 38.9255 37.465) (end 36.957 37.465) (width 0.25) (layer F.Cu) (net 3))
 (segment (start 37.4015 31.369) (end 36.195 31.369) (width 0.25) (layer F.Cu) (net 2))
 (segment (start 37.592 31.5595) (end 37.4015 31.369) (width 0.25) (layer F.Cu) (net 2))
 (segment (start 37.592 32.512) (end 37.592 31.5595) (width 0.25) (layer F.Cu) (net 2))
 (segment (start 38.96 32.807) (end 37.887 32.807) (width 0.25) (layer F.Cu) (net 2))
 (segment (start 37.887 32.807) (end 37.592 32.512) (width 0.25) (layer F.Cu) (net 2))
 (segment (start 36.957 38.608) (end 36.957 40.1955) (width 0.25) (layer F.Cu) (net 2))
 (segment (start 40.7445 32.807) (end 41.2115 33.274) (width 0.25) (layer F.Cu) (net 2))
 (segment (start 41.2115 33.274) (end 41.2115 36.322) (width 0.25) (layer F.Cu) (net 2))
 (segment (start 37.465 38.1) (end 36.957 38.608) (width 0.25) (layer F.Cu) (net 2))
 (segment (start 38.96 32.807) (end 40.7445 32.807) (width 0.25) (layer F.Cu) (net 2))
 (segment (start 39.4335 38.1) (end 37.465 38.1) (width 0.25) (layer F.Cu) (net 2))
 (segment (start 41.2115 36.322) (end 39.4335 38.1) (width 0.25) (layer F.Cu) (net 2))
 (segment (start 39.497 40.1955) (end 39.497 39.1795) (width 0.25) (layer F.Cu) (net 7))
 (segment (start 39.497 39.1795) (end 42.672 36.0045) (width 0.25) (layer F.Cu) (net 7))
 (segment (start 42.672 36.0045) (end 42.672 33.8455) (width 0.25) (layer F.Cu) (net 7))
 (segment (start 43.0605 33.457) (end 44.86 33.457) (width 0.25) (layer F.Cu) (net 7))
 (segment (start 42.672 33.8455) (end 43.0605 33.457) (width 0.25) (layer F.Cu) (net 7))
 (segment (start 28.6385 33.368) (end 30.988 33.368) (width 0.25) (layer F.Cu) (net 9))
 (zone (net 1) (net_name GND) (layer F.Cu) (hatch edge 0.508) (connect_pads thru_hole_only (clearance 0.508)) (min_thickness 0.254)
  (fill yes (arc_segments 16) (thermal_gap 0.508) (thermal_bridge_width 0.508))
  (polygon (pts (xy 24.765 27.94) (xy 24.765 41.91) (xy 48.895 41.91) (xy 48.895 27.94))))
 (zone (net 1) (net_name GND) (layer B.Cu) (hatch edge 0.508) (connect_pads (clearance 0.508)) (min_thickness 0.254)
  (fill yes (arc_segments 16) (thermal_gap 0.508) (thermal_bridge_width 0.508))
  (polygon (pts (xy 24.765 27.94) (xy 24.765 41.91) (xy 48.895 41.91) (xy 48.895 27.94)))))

